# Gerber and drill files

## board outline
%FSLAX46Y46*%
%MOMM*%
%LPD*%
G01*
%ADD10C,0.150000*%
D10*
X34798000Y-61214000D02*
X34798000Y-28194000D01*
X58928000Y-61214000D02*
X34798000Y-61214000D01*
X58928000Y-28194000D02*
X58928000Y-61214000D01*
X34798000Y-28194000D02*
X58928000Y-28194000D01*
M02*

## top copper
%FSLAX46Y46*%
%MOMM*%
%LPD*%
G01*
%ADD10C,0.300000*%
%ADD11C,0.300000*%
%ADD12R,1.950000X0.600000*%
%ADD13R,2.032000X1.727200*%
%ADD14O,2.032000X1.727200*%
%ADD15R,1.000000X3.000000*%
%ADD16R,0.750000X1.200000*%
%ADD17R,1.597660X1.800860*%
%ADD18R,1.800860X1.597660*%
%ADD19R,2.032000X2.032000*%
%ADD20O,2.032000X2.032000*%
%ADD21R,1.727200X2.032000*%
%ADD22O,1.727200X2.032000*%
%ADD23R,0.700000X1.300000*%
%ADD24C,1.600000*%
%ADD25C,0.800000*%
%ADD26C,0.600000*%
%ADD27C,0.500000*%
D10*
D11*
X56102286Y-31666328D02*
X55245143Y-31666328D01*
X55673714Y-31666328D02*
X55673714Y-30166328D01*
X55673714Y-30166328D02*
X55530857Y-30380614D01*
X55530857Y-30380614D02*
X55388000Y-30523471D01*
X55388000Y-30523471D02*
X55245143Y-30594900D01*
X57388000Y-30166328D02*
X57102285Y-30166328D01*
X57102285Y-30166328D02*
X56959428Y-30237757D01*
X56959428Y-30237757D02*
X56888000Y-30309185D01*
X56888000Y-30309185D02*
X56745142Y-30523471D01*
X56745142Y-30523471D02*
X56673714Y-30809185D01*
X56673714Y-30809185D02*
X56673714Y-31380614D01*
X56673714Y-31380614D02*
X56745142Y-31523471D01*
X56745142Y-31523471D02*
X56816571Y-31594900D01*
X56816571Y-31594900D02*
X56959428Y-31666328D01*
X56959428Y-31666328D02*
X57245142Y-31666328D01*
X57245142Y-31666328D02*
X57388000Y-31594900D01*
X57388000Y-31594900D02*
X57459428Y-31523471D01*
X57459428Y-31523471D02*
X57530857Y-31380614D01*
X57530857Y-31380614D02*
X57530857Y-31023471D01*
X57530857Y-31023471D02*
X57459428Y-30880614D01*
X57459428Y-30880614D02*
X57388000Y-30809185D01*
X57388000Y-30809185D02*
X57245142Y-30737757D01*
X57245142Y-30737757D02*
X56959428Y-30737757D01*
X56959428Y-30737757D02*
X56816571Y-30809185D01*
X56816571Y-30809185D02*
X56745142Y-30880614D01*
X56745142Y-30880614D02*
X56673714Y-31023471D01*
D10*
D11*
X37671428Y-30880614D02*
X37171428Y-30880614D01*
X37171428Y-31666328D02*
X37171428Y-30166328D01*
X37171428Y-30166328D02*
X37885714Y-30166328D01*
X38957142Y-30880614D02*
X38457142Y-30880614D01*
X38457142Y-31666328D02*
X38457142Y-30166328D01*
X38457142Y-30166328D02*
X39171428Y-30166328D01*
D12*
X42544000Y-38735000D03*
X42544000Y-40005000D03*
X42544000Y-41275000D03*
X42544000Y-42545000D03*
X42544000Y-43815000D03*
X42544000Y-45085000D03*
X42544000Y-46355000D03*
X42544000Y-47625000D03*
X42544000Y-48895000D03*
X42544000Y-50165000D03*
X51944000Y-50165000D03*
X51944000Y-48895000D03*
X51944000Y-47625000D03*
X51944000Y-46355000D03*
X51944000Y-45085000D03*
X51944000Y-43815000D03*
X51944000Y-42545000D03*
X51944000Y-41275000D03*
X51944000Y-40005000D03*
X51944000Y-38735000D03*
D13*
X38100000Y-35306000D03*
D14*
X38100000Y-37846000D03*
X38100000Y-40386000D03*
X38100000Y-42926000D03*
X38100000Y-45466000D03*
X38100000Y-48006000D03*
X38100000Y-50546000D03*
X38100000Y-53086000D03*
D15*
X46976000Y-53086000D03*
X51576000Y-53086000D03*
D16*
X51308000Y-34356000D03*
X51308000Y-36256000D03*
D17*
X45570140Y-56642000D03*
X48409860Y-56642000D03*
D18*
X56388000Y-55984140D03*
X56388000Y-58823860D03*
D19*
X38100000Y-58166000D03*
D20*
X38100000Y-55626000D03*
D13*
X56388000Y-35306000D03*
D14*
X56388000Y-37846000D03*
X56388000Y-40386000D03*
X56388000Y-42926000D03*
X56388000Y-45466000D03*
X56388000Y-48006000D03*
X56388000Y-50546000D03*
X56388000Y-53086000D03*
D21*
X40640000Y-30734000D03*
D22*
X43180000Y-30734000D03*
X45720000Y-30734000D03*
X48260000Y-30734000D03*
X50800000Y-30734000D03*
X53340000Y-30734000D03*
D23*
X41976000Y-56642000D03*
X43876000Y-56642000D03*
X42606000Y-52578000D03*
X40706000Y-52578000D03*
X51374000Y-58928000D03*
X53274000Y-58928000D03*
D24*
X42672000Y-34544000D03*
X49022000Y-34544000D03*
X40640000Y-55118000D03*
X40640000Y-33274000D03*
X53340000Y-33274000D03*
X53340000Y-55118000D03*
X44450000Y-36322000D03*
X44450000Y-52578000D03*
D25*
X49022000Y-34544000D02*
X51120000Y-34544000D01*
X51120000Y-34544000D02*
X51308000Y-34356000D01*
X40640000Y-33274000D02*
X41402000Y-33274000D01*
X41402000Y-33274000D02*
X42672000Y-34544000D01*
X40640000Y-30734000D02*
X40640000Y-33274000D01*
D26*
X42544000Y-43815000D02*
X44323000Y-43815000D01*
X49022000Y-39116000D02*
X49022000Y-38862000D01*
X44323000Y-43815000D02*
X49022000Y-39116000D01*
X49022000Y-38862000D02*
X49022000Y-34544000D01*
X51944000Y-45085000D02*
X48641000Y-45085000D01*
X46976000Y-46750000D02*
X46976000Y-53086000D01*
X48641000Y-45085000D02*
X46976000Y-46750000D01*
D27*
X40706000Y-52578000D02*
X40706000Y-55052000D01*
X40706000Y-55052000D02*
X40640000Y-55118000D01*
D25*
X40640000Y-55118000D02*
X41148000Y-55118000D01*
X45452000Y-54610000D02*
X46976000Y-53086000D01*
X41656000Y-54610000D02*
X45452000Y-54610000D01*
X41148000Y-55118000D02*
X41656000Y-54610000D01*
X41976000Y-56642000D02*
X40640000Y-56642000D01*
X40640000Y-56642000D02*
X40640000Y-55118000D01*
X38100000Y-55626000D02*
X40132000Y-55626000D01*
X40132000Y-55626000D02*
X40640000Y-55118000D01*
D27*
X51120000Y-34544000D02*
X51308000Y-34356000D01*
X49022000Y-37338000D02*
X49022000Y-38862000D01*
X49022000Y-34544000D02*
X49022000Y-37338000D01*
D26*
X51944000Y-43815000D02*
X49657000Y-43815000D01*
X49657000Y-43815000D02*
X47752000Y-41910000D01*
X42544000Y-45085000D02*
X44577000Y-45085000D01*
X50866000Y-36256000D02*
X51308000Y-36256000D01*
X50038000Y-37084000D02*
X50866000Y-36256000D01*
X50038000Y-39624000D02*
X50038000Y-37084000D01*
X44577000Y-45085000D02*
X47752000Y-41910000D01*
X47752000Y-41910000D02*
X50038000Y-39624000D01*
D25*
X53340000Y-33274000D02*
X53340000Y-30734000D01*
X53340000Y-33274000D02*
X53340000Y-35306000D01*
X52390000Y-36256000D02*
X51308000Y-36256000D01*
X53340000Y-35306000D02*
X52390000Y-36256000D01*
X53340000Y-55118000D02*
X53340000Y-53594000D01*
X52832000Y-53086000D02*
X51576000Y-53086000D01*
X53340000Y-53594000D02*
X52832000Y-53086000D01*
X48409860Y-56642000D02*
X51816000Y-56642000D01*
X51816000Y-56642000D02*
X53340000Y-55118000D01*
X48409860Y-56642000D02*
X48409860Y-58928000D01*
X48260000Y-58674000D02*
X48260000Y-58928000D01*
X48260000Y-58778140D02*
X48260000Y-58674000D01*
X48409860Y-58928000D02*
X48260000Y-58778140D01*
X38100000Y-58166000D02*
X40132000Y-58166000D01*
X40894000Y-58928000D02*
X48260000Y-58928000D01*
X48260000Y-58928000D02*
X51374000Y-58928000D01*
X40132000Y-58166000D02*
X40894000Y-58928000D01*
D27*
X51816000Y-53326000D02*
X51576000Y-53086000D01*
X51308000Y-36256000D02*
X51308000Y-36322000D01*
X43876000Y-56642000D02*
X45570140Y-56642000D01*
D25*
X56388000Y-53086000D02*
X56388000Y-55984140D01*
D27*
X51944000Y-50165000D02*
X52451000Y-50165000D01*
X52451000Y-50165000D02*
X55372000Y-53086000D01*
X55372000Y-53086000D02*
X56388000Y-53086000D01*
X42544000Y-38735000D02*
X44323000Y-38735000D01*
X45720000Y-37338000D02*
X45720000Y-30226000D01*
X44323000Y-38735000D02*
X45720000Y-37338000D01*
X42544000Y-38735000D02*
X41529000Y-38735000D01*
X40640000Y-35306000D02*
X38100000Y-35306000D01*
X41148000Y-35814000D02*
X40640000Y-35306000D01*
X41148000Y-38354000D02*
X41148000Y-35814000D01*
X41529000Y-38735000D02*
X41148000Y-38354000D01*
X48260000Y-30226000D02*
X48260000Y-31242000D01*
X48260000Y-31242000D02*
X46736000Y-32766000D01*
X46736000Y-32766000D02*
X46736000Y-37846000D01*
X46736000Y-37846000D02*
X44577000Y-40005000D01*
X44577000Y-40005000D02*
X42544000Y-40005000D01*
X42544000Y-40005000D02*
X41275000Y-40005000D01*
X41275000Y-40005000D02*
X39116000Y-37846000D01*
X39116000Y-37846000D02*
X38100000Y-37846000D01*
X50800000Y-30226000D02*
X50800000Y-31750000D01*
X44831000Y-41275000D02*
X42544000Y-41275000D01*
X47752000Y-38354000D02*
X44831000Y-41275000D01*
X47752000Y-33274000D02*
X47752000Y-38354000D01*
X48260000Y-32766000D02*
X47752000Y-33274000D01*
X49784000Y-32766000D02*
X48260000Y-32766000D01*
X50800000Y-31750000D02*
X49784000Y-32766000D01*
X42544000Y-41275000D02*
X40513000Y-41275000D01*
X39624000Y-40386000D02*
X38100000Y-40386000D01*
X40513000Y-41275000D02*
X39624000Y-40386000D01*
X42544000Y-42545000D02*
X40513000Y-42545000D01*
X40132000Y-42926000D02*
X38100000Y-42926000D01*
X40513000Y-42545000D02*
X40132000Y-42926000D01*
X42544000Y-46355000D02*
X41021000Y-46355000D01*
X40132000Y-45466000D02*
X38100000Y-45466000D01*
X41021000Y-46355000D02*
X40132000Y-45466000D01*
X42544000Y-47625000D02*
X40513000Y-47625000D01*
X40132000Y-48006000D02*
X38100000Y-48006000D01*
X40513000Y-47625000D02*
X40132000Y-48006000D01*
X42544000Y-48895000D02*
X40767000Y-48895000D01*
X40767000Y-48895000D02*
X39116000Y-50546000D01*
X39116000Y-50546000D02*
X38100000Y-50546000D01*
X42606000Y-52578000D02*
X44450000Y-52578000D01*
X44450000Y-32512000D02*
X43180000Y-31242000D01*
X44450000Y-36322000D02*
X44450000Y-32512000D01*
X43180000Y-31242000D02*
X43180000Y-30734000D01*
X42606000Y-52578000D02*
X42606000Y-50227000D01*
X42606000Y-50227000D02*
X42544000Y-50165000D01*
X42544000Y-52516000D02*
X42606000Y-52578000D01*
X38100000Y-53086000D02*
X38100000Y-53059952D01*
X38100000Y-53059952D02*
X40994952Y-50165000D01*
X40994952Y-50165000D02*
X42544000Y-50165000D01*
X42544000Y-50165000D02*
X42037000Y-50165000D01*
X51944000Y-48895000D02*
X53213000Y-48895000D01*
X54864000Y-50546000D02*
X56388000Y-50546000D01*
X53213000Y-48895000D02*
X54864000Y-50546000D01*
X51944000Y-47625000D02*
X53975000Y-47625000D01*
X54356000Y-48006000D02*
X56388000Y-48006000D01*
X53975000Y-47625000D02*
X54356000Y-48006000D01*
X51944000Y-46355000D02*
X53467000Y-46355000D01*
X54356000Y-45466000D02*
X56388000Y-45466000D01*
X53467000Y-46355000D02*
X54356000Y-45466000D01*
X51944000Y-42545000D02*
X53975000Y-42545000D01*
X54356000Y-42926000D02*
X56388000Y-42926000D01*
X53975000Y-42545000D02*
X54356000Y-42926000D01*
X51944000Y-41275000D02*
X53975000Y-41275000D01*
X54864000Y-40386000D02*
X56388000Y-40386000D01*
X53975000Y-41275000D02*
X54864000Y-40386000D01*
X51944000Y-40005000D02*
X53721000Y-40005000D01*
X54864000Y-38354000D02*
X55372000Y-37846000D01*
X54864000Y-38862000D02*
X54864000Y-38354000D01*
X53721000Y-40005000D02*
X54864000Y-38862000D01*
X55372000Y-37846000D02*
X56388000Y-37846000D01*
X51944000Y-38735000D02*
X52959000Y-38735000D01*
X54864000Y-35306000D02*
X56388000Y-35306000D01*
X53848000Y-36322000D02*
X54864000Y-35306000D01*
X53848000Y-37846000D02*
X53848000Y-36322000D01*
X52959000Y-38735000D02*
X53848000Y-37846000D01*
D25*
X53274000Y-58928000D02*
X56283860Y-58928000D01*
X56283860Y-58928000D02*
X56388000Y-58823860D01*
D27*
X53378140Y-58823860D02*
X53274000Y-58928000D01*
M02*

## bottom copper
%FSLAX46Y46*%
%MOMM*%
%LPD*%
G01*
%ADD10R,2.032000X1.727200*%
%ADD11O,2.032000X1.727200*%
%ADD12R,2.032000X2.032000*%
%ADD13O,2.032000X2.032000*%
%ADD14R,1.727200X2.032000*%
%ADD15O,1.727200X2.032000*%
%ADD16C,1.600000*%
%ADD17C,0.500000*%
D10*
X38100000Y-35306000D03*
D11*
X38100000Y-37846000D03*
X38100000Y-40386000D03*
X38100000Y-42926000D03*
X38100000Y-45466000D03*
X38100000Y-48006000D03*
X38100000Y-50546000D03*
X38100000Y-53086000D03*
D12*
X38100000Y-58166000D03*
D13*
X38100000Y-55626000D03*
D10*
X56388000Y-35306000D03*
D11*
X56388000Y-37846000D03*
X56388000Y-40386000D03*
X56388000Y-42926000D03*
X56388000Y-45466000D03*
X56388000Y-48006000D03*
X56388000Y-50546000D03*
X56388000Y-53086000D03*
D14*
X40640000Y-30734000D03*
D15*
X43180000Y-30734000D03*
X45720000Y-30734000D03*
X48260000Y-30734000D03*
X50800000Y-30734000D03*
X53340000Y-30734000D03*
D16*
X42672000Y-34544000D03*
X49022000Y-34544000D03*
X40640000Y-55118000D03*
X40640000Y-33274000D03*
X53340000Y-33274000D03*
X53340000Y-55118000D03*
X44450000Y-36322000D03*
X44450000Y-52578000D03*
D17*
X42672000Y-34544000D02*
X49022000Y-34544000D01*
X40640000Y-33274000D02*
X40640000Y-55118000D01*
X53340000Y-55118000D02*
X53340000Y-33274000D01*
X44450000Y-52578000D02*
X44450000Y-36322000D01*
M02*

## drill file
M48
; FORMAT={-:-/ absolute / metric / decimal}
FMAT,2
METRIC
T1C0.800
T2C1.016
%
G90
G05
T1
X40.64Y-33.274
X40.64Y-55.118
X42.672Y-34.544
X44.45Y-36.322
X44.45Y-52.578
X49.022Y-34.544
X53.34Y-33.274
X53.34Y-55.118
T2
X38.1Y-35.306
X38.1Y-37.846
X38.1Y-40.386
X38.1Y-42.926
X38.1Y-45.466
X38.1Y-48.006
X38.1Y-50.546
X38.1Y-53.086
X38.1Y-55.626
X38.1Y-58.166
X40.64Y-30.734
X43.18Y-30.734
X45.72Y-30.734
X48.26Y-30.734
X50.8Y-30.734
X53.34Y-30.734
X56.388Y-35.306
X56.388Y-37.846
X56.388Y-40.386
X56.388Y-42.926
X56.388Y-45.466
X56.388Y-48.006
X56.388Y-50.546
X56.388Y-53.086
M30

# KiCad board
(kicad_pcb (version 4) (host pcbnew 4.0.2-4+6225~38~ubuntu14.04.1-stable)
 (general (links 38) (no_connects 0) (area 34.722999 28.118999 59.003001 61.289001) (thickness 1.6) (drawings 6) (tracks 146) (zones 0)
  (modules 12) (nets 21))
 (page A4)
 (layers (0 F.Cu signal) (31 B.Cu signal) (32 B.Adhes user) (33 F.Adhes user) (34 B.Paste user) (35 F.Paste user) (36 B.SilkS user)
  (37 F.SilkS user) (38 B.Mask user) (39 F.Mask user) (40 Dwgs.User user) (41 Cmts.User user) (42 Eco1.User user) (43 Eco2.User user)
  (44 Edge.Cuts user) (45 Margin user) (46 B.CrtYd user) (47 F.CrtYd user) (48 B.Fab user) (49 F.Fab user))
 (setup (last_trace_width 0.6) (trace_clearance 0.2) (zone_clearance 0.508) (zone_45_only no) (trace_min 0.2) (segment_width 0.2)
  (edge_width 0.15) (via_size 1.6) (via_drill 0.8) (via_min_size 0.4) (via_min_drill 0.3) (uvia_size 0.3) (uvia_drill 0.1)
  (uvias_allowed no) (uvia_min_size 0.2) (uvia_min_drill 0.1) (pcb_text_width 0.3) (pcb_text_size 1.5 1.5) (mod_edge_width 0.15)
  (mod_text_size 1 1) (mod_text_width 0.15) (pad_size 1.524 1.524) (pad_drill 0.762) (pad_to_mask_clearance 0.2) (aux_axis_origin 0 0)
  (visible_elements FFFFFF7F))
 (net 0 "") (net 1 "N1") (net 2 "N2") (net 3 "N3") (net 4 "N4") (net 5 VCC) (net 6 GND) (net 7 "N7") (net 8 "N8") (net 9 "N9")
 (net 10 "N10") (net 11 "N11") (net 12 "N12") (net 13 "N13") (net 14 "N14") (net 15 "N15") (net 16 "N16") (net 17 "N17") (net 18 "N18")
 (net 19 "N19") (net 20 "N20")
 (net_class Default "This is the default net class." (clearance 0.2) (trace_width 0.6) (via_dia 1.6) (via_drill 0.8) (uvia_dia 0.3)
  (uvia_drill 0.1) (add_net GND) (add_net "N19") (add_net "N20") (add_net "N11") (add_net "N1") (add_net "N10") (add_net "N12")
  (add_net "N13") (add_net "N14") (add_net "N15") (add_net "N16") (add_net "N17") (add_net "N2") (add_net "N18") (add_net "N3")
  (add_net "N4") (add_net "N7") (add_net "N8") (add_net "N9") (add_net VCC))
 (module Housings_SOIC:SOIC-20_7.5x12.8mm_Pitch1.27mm (layer F.Cu) (at 47.244 44.45)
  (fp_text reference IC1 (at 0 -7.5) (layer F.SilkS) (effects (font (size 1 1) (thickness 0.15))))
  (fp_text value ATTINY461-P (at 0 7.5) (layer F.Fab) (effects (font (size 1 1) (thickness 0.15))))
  (pad 1 smd rect (at -4.7 -5.715) (size 1.95 0.6) (layers F.Cu F.Paste F.Mask) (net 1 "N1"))
  (pad 2 smd rect (at -4.7 -4.445) (size 1.95 0.6) (layers F.Cu F.Paste F.Mask) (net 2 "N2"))
  (pad 3 smd rect (at -4.7 -3.175) (size 1.95 0.6) (layers F.Cu F.Paste F.Mask) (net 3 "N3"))
  (pad 4 smd rect (at -4.7 -1.905) (size 1.95 0.6) (layers F.Cu F.Paste F.Mask) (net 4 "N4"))
  (pad 5 smd rect (at -4.7 -0.635) (size 1.95 0.6) (layers F.Cu F.Paste F.Mask) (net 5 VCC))
  (pad 6 smd rect (at -4.7 0.635) (size 1.95 0.6) (layers F.Cu F.Paste F.Mask) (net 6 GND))
  (pad 7 smd rect (at -4.7 1.905) (size 1.95 0.6) (layers F.Cu F.Paste F.Mask) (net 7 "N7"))
  (pad 8 smd rect (at -4.7 3.175) (size 1.95 0.6) (layers F.Cu F.Paste F.Mask) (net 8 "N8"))
  (pad 9 smd rect (at -4.7 4.445) (size 1.95 0.6) (layers F.Cu F.Paste F.Mask) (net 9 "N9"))
  (pad 10 smd rect (at -4.7 5.715) (size 1.95 0.6) (layers F.Cu F.Paste F.Mask) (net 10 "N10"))
  (pad 11 smd rect (at 4.7 5.715) (size 1.95 0.6) (layers F.Cu F.Paste F.Mask) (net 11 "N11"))
  (pad 12 smd rect (at 4.7 4.445) (size 1.95 0.6) (layers F.Cu F.Paste F.Mask) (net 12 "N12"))
  (pad 13 smd rect (at 4.7 3.175) (size 1.95 0.6) (layers F.Cu F.Paste F.Mask) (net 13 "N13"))
  (pad 14 smd rect (at 4.7 1.905) (size 1.95 0.6) (layers F.Cu F.Paste F.Mask) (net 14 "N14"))
  (pad 15 smd rect (at 4.7 0.635) (size 1.95 0.6) (layers F.Cu F.Paste F.Mask) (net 5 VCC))
  (pad 16 smd rect (at 4.7 -0.635) (size 1.95 0.6) (layers F.Cu F.Paste F.Mask) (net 6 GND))
  (pad 17 smd rect (at 4.7 -1.905) (size 1.95 0.6) (layers F.Cu F.Paste F.Mask) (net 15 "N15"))
  (pad 18 smd rect (at 4.7 -3.175) (size 1.95 0.6) (layers F.Cu F.Paste F.Mask) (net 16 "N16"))
  (pad 19 smd rect (at 4.7 -4.445) (size 1.95 0.6) (layers F.Cu F.Paste F.Mask) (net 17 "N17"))
  (pad 20 smd rect (at 4.7 -5.715) (size 1.95 0.6) (layers F.Cu F.Paste F.Mask) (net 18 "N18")))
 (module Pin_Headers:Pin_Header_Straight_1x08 (layer F.Cu) (at 38.1 35.306)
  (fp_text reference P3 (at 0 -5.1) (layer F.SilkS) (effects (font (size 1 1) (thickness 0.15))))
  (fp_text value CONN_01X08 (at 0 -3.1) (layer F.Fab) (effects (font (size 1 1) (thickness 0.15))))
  (pad 1 thru_hole rect (at 0 0) (size 2.032 1.7272) (drill 1.016) (layers *.Cu *.Mask F.SilkS) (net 1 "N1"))
  (pad 2 thru_hole oval (at 0 2.54) (size 2.032 1.7272) (drill 1.016) (layers *.Cu *.Mask F.SilkS) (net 2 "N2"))
  (pad 3 thru_hole oval (at 0 5.08) (size 2.032 1.7272) (drill 1.016) (layers *.Cu *.Mask F.SilkS) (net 3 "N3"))
  (pad 4 thru_hole oval (at 0 7.62) (size 2.032 1.7272) (drill 1.016) (layers *.Cu *.Mask F.SilkS) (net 4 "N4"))
  (pad 5 thru_hole oval (at 0 10.16) (size 2.032 1.7272) (drill 1.016) (layers *.Cu *.Mask F.SilkS) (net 7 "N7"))
  (pad 6 thru_hole oval (at 0 12.7) (size 2.032 1.7272) (drill 1.016) (layers *.Cu *.Mask F.SilkS) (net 8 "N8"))
  (pad 7 thru_hole oval (at 0 15.24) (size 2.032 1.7272) (drill 1.016) (layers *.Cu *.Mask F.SilkS) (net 9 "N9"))
  (pad 8 thru_hole oval (at 0 17.78) (size 2.032 1.7272) (drill 1.016) (layers *.Cu *.Mask F.SilkS) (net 10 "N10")))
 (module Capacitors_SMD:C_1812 (layer F.Cu) (at 49.276 53.086)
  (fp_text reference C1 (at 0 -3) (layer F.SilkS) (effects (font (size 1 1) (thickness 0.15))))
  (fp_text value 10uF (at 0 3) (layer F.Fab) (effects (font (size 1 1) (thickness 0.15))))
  (pad 1 smd rect (at -2.3 0) (size 1 3) (layers F.Cu F.Paste F.Mask) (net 5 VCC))
  (pad 2 smd rect (at 2.3 0) (size 1 3) (layers F.Cu F.Paste F.Mask) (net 6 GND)))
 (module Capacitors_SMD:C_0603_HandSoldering (layer F.Cu) (at 51.308 35.306 270)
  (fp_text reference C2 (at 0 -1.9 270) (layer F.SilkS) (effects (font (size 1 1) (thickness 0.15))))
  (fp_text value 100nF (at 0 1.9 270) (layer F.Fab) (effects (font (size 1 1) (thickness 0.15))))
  (pad 1 smd rect (at -0.95 0 270) (size 1.2 0.75) (layers F.Cu F.Paste F.Mask) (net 5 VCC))
  (pad 2 smd rect (at 0.95 0 270) (size 1.2 0.75) (layers F.Cu F.Paste F.Mask) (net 6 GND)))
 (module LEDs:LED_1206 (layer F.Cu) (at 46.99 56.642 180)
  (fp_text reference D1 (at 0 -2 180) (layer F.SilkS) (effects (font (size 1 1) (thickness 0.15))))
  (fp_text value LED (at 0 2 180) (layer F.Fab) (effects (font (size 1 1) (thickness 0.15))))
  (pad 2 smd rect (at 1.41986 0) (size 1.59766 1.80086) (layers F.Cu F.Paste F.Mask) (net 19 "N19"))
  (pad 1 smd rect (at -1.41986 0) (size 1.59766 1.80086) (layers F.Cu F.Paste F.Mask) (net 6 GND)))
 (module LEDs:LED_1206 (layer F.Cu) (at 56.388 57.404 90)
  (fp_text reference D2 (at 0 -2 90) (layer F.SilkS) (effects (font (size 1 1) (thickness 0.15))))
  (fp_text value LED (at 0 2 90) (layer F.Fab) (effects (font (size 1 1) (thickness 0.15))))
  (pad 2 smd rect (at 1.41986 0 270) (size 1.59766 1.80086) (layers F.Cu F.Paste F.Mask) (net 11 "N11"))
  (pad 1 smd rect (at -1.41986 0 270) (size 1.59766 1.80086) (layers F.Cu F.Paste F.Mask) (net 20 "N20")))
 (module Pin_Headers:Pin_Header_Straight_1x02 (layer F.Cu) (at 38.1 58.166 180)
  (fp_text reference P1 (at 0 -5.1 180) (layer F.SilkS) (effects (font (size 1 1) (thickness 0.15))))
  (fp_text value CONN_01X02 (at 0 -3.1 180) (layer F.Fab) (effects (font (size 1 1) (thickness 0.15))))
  (pad 1 thru_hole rect (at 0 0 180) (size 2.032 2.032) (drill 1.016) (layers *.Cu *.Mask F.SilkS) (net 6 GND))
  (pad 2 thru_hole oval (at 0 2.54 180) (size 2.032 2.032) (drill 1.016) (layers *.Cu *.Mask F.SilkS) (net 5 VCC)))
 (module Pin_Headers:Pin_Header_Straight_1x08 (layer F.Cu) (at 56.388 35.306)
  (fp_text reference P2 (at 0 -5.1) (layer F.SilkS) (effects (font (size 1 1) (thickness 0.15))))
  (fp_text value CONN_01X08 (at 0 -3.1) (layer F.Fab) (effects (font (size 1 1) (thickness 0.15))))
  (pad 1 thru_hole rect (at 0 0) (size 2.032 1.7272) (drill 1.016) (layers *.Cu *.Mask F.SilkS) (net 18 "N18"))
  (pad 2 thru_hole oval (at 0 2.54) (size 2.032 1.7272) (drill 1.016) (layers *.Cu *.Mask F.SilkS) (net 17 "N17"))
  (pad 3 thru_hole oval (at 0 5.08) (size 2.032 1.7272) (drill 1.016) (layers *.Cu *.Mask F.SilkS) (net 16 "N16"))
  (pad 4 thru_hole oval (at 0 7.62) (size 2.032 1.7272) (drill 1.016) (layers *.Cu *.Mask F.SilkS) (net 15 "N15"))
  (pad 5 thru_hole oval (at 0 10.16) (size 2.032 1.7272) (drill 1.016) (layers *.Cu *.Mask F.SilkS) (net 14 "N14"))
  (pad 6 thru_hole oval (at 0 12.7) (size 2.032 1.7272) (drill 1.016) (layers *.Cu *.Mask F.SilkS) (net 13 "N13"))
  (pad 7 thru_hole oval (at 0 15.24) (size 2.032 1.7272) (drill 1.016) (layers *.Cu *.Mask F.SilkS) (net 12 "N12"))
  (pad 8 thru_hole oval (at 0 17.78) (size 2.032 1.7272) (drill 1.016) (layers *.Cu *.Mask F.SilkS) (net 11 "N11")))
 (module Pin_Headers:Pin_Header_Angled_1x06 (layer F.Cu) (at 40.64 30.734 90)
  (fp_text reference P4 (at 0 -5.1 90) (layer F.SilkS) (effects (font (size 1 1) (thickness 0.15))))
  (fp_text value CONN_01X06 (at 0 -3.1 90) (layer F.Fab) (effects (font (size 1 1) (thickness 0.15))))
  (pad 1 thru_hole rect (at 0 0 90) (size 2.032 1.7272) (drill 1.016) (layers *.Cu *.Mask F.SilkS) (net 5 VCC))
  (pad 2 thru_hole oval (at 0 2.54 90) (size 2.032 1.7272) (drill 1.016) (layers *.Cu *.Mask F.SilkS) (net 10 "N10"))
  (pad 3 thru_hole oval (at 0 5.08 90) (size 2.032 1.7272) (drill 1.016) (layers *.Cu *.Mask F.SilkS) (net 1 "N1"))
  (pad 4 thru_hole oval (at 0 7.62 90) (size 2.032 1.7272) (drill 1.016) (layers *.Cu *.Mask F.SilkS) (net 2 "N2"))
  (pad 5 thru_hole oval (at 0 10.16 90) (size 2.032 1.7272) (drill 1.016) (layers *.Cu *.Mask F.SilkS) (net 3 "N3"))
  (pad 6 thru_hole oval (at 0 12.7 90) (size 2.032 1.7272) (drill 1.016) (layers *.Cu *.Mask F.SilkS) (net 6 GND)))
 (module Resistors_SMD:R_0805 (layer F.Cu) (at 42.926 56.642)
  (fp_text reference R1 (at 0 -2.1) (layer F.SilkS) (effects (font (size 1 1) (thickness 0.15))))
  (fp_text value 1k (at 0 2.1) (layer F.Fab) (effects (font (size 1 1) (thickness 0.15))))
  (pad 1 smd rect (at -0.95 0) (size 0.7 1.3) (layers F.Cu F.Paste F.Mask) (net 5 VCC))
  (pad 2 smd rect (at 0.95 0) (size 0.7 1.3) (layers F.Cu F.Paste F.Mask) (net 19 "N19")))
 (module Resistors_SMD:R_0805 (layer F.Cu) (at 41.656 52.578 180)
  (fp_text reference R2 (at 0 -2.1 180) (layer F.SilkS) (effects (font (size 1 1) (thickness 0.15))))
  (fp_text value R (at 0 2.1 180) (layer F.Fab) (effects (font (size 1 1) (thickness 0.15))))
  (pad 1 smd rect (at -0.95 0 180) (size 0.7 1.3) (layers F.Cu F.Paste F.Mask) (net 10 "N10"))
  (pad 2 smd rect (at 0.95 0 180) (size 0.7 1.3) (layers F.Cu F.Paste F.Mask) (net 5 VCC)))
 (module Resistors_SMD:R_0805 (layer F.Cu) (at 52.324 58.928)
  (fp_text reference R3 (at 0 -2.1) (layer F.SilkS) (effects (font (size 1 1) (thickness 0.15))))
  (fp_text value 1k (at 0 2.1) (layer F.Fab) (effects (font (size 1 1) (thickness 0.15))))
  (pad 1 smd rect (at -0.95 0) (size 0.7 1.3) (layers F.Cu F.Paste F.Mask) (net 6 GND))
  (pad 2 smd rect (at 0.95 0) (size 0.7 1.3) (layers F.Cu F.Paste F.Mask) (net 20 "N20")))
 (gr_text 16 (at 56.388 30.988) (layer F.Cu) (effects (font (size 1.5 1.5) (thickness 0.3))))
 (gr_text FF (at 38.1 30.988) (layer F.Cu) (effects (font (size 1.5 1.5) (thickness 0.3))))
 (gr_line (start 34.798 61.214) (end 34.798 28.194) (angle 90) (layer Edge.Cuts) (width 0.15))
 (gr_line (start 58.928 61.214) (end 34.798 61.214) (angle 90) (layer Edge.Cuts) (width 0.15))
 (gr_line (start 58.928 28.194) (end 58.928 61.214) (angle 90) (layer Edge.Cuts) (width 0.15))
 (gr_line (start 34.798 28.194) (end 58.928 28.194) (angle 90) (layer Edge.Cuts) (width 0.15))
 (segment (start 49.022 34.544) (end 51.12 34.544) (width 0.8) (layer F.Cu) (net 5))
 (segment (start 51.12 34.544) (end 51.308 34.356) (width 0.8) (layer F.Cu) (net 5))
 (segment (start 40.64 33.274) (end 41.402 33.274) (width 0.8) (layer F.Cu) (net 5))
 (segment (start 42.672 34.544) (end 49.022 34.544) (width 0.5) (layer B.Cu) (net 5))
 (segment (start 41.402 33.274) (end 42.672 34.544) (width 0.8) (layer F.Cu) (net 5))
 (segment (start 40.64 30.734) (end 40.64 33.274) (width 0.8) (layer F.Cu) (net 5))
 (segment (start 40.64 33.274) (end 40.64 55.118) (width 0.5) (layer B.Cu) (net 5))
 (segment (start 42.544 43.815) (end 44.323 43.815) (width 0.6) (layer F.Cu) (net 5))
 (segment (start 49.022 39.116) (end 49.022 38.862) (width 0.6) (layer F.Cu) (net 5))
 (segment (start 44.323 43.815) (end 49.022 39.116) (width 0.6) (layer F.Cu) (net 5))
 (segment (start 49.022 38.862) (end 49.022 34.544) (width 0.6) (layer F.Cu) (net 5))
 (segment (start 51.944 45.085) (end 48.641 45.085) (width 0.6) (layer F.Cu) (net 5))
 (segment (start 46.976 46.75) (end 46.976 53.086) (width 0.6) (layer F.Cu) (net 5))
 (segment (start 48.641 45.085) (end 46.976 46.75) (width 0.6) (layer F.Cu) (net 5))
 (segment (start 40.706 52.578) (end 40.706 55.052) (width 0.5) (layer F.Cu) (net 5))
 (segment (start 40.706 55.052) (end 40.64 55.118) (width 0.5) (layer F.Cu) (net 5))
 (segment (start 40.64 55.118) (end 41.148 55.118) (width 0.8) (layer F.Cu) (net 5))
 (segment (start 45.452 54.61) (end 46.976 53.086) (width 0.8) (layer F.Cu) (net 5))
 (segment (start 41.656 54.61) (end 45.452 54.61) (width 0.8) (layer F.Cu) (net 5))
 (segment (start 41.148 55.118) (end 41.656 54.61) (width 0.8) (layer F.Cu) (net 5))
 (segment (start 41.976 56.642) (end 40.64 56.642) (width 0.8) (layer F.Cu) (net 5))
 (segment (start 40.64 56.642) (end 40.64 55.118) (width 0.8) (layer F.Cu) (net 5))
 (segment (start 38.1 55.626) (end 40.132 55.626) (width 0.8) (layer F.Cu) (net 5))
 (segment (start 40.132 55.626) (end 40.64 55.118) (width 0.8) (layer F.Cu) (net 5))
 (segment (start 51.12 34.544) (end 51.308 34.356) (width 0.5) (layer F.Cu) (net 5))
 (segment (start 49.022 37.338) (end 49.022 38.862) (width 0.5) (layer F.Cu) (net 5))
 (segment (start 49.022 34.544) (end 49.022 37.338) (width 0.5) (layer F.Cu) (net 5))
 (segment (start 51.944 43.815) (end 49.657 43.815) (width 0.6) (layer F.Cu) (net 6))
 (segment (start 49.657 43.815) (end 47.752 41.91) (width 0.6) (layer F.Cu) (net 6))
 (segment (start 42.544 45.085) (end 44.577 45.085) (width 0.6) (layer F.Cu) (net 6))
 (segment (start 50.866 36.256) (end 51.308 36.256) (width 0.6) (layer F.Cu) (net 6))
 (segment (start 50.038 37.084) (end 50.866 36.256) (width 0.6) (layer F.Cu) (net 6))
 (segment (start 50.038 39.624) (end 50.038 37.084) (width 0.6) (layer F.Cu) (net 6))
 (segment (start 44.577 45.085) (end 47.752 41.91) (width 0.6) (layer F.Cu) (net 6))
 (segment (start 47.752 41.91) (end 50.038 39.624) (width 0.6) (layer F.Cu) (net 6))
 (segment (start 53.34 33.274) (end 53.34 30.734) (width 0.8) (layer F.Cu) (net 6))
 (segment (start 53.34 33.274) (end 53.34 35.306) (width 0.8) (layer F.Cu) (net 6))
 (segment (start 53.34 55.118) (end 53.34 33.274) (width 0.5) (layer B.Cu) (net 6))
 (segment (start 52.39 36.256) (end 51.308 36.256) (width 0.8) (layer F.Cu) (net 6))
 (segment (start 53.34 35.306) (end 52.39 36.256) (width 0.8) (layer F.Cu) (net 6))
 (segment (start 53.34 55.118) (end 53.34 53.594) (width 0.8) (layer F.Cu) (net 6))
 (segment (start 52.832 53.086) (end 51.576 53.086) (width 0.8) (layer F.Cu) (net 6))
 (segment (start 53.34 53.594) (end 52.832 53.086) (width 0.8) (layer F.Cu) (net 6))
 (segment (start 48.40986 56.642) (end 51.816 56.642) (width 0.8) (layer F.Cu) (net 6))
 (segment (start 51.816 56.642) (end 53.34 55.118) (width 0.8) (layer F.Cu) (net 6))
 (segment (start 48.40986 56.642) (end 48.40986 58.928) (width 0.8) (layer F.Cu) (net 6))
 (segment (start 48.26 58.674) (end 48.26 58.928) (width 0.8) (layer F.Cu) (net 6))
 (segment (start 48.26 58.77814) (end 48.26 58.674) (width 0.8) (layer F.Cu) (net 6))
 (segment (start 48.40986 58.928) (end 48.26 58.77814) (width 0.8) (layer F.Cu) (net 6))
 (segment (start 38.1 58.166) (end 40.132 58.166) (width 0.8) (layer F.Cu) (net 6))
 (segment (start 40.894 58.928) (end 48.26 58.928) (width 0.8) (layer F.Cu) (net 6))
 (segment (start 48.26 58.928) (end 51.374 58.928) (width 0.8) (layer F.Cu) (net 6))
 (segment (start 40.132 58.166) (end 40.894 58.928) (width 0.8) (layer F.Cu) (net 6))
 (segment (start 51.816 53.326) (end 51.576 53.086) (width 0.5) (layer F.Cu) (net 6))
 (segment (start 51.308 36.256) (end 51.308 36.322) (width 0.5) (layer F.Cu) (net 6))
 (segment (start 43.876 56.642) (end 45.57014 56.642) (width 0.5) (layer F.Cu) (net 19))
 (segment (start 56.388 53.086) (end 56.388 55.98414) (width 0.8) (layer F.Cu) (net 11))
 (segment (start 51.944 50.165) (end 52.451 50.165) (width 0.5) (layer F.Cu) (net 11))
 (segment (start 52.451 50.165) (end 55.372 53.086) (width 0.5) (layer F.Cu) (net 11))
 (segment (start 55.372 53.086) (end 56.388 53.086) (width 0.5) (layer F.Cu) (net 11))
 (segment (start 42.544 38.735) (end 44.323 38.735) (width 0.5) (layer F.Cu) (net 1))
 (segment (start 45.72 37.338) (end 45.72 30.226) (width 0.5) (layer F.Cu) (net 1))
 (segment (start 44.323 38.735) (end 45.72 37.338) (width 0.5) (layer F.Cu) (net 1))
 (segment (start 42.544 38.735) (end 41.529 38.735) (width 0.5) (layer F.Cu) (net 1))
 (segment (start 40.64 35.306) (end 38.1 35.306) (width 0.5) (layer F.Cu) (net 1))
 (segment (start 41.148 35.814) (end 40.64 35.306) (width 0.5) (layer F.Cu) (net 1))
 (segment (start 41.148 38.354) (end 41.148 35.814) (width 0.5) (layer F.Cu) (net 1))
 (segment (start 41.529 38.735) (end 41.148 38.354) (width 0.5) (layer F.Cu) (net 1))
 (segment (start 48.26 30.226) (end 48.26 31.242) (width 0.5) (layer F.Cu) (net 2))
 (segment (start 48.26 31.242) (end 46.736 32.766) (width 0.5) (layer F.Cu) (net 2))
 (segment (start 46.736 32.766) (end 46.736 37.846) (width 0.5) (layer F.Cu) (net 2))
 (segment (start 46.736 37.846) (end 44.577 40.005) (width 0.5) (layer F.Cu) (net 2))
 (segment (start 44.577 40.005) (end 42.544 40.005) (width 0.5) (layer F.Cu) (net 2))
 (segment (start 42.544 40.005) (end 41.275 40.005) (width 0.5) (layer F.Cu) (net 2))
 (segment (start 41.275 40.005) (end 39.116 37.846) (width 0.5) (layer F.Cu) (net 2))
 (segment (start 39.116 37.846) (end 38.1 37.846) (width 0.5) (layer F.Cu) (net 2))
 (segment (start 50.8 30.226) (end 50.8 31.75) (width 0.5) (layer F.Cu) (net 3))
 (segment (start 44.831 41.275) (end 42.544 41.275) (width 0.5) (layer F.Cu) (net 3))
 (segment (start 47.752 38.354) (end 44.831 41.275) (width 0.5) (layer F.Cu) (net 3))
 (segment (start 47.752 33.274) (end 47.752 38.354) (width 0.5) (layer F.Cu) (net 3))
 (segment (start 48.26 32.766) (end 47.752 33.274) (width 0.5) (layer F.Cu) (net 3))
 (segment (start 49.784 32.766) (end 48.26 32.766) (width 0.5) (layer F.Cu) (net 3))
 (segment (start 50.8 31.75) (end 49.784 32.766) (width 0.5) (layer F.Cu) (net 3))
 (segment (start 42.544 41.275) (end 40.513 41.275) (width 0.5) (layer F.Cu) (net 3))
 (segment (start 39.624 40.386) (end 38.1 40.386) (width 0.5) (layer F.Cu) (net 3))
 (segment (start 40.513 41.275) (end 39.624 40.386) (width 0.5) (layer F.Cu) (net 3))
 (segment (start 42.544 42.545) (end 40.513 42.545) (width 0.5) (layer F.Cu) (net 4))
 (segment (start 40.132 42.926) (end 38.1 42.926) (width 0.5) (layer F.Cu) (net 4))
 (segment (start 40.513 42.545) (end 40.132 42.926) (width 0.5) (layer F.Cu) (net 4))
 (segment (start 42.544 46.355) (end 41.021 46.355) (width 0.5) (layer F.Cu) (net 7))
 (segment (start 40.132 45.466) (end 38.1 45.466) (width 0.5) (layer F.Cu) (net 7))
 (segment (start 41.021 46.355) (end 40.132 45.466) (width 0.5) (layer F.Cu) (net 7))
 (segment (start 42.544 47.625) (end 40.513 47.625) (width 0.5) (layer F.Cu) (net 8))
 (segment (start 40.132 48.006) (end 38.1 48.006) (width 0.5) (layer F.Cu) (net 8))
 (segment (start 40.513 47.625) (end 40.132 48.006) (width 0.5) (layer F.Cu) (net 8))
 (segment (start 42.544 48.895) (end 40.767 48.895) (width 0.5) (layer F.Cu) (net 9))
 (segment (start 40.767 48.895) (end 39.116 50.546) (width 0.5) (layer F.Cu) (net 9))
 (segment (start 39.116 50.546) (end 38.1 50.546) (width 0.5) (layer F.Cu) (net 9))
 (segment (start 42.606 52.578) (end 44.45 52.578) (width 0.5) (layer F.Cu) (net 10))
 (segment (start 44.45 32.512) (end 43.18 31.242) (width 0.5) (layer F.Cu) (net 10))
 (segment (start 44.45 36.322) (end 44.45 32.512) (width 0.5) (layer F.Cu) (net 10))
 (segment (start 44.45 52.578) (end 44.45 36.322) (width 0.5) (layer B.Cu) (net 10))
 (segment (start 43.18 31.242) (end 43.18 30.734) (width 0.5) (layer F.Cu) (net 10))
 (segment (start 42.606 52.578) (end 42.606 50.227) (width 0.5) (layer F.Cu) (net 10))
 (segment (start 42.606 50.227) (end 42.544 50.165) (width 0.5) (layer F.Cu) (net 10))
 (segment (start 42.544 52.516) (end 42.606 52.578) (width 0.5) (layer F.Cu) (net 10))
 (segment (start 38.1 53.086) (end 38.1 53.059952) (width 0.5) (layer F.Cu) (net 10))
 (segment (start 38.1 53.059952) (end 40.994952 50.165) (width 0.5) (layer F.Cu) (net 10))
 (segment (start 40.994952 50.165) (end 42.544 50.165) (width 0.5) (layer F.Cu) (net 10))
 (segment (start 42.544 50.165) (end 42.037 50.165) (width 0.5) (layer F.Cu) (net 10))
 (segment (start 51.944 48.895) (end 53.213 48.895) (width 0.5) (layer F.Cu) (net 12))
 (segment (start 54.864 50.546) (end 56.388 50.546) (width 0.5) (layer F.Cu) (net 12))
 (segment (start 53.213 48.895) (end 54.864 50.546) (width 0.5) (layer F.Cu) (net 12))
 (segment (start 51.944 47.625) (end 53.975 47.625) (width 0.5) (layer F.Cu) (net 13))
 (segment (start 54.356 48.006) (end 56.388 48.006) (width 0.5) (layer F.Cu) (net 13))
 (segment (start 53.975 47.625) (end 54.356 48.006) (width 0.5) (layer F.Cu) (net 13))
 (segment (start 51.944 46.355) (end 53.467 46.355) (width 0.5) (layer F.Cu) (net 14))
 (segment (start 54.356 45.466) (end 56.388 45.466) (width 0.5) (layer F.Cu) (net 14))
 (segment (start 53.467 46.355) (end 54.356 45.466) (width 0.5) (layer F.Cu) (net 14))
 (segment (start 51.944 42.545) (end 53.975 42.545) (width 0.5) (layer F.Cu) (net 15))
 (segment (start 54.356 42.926) (end 56.388 42.926) (width 0.5) (layer F.Cu) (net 15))
 (segment (start 53.975 42.545) (end 54.356 42.926) (width 0.5) (layer F.Cu) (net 15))
 (segment (start 51.944 41.275) (end 53.975 41.275) (width 0.5) (layer F.Cu) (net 16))
 (segment (start 54.864 40.386) (end 56.388 40.386) (width 0.5) (layer F.Cu) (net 16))
 (segment (start 53.975 41.275) (end 54.864 40.386) (width 0.5) (layer F.Cu) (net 16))
 (segment (start 51.944 40.005) (end 53.721 40.005) (width 0.5) (layer F.Cu) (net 17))
 (segment (start 54.864 38.354) (end 55.372 37.846) (width 0.5) (layer F.Cu) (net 17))
 (segment (start 54.864 38.862) (end 54.864 38.354) (width 0.5) (layer F.Cu) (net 17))
 (segment (start 53.721 40.005) (end 54.864 38.862) (width 0.5) (layer F.Cu) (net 17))
 (segment (start 55.372 37.846) (end 56.388 37.846) (width 0.5) (layer F.Cu) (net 17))
 (segment (start 51.944 38.735) (end 52.959 38.735) (width 0.5) (layer F.Cu) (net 18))
 (segment (start 54.864 35.306) (end 56.388 35.306) (width 0.5) (layer F.Cu) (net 18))
 (segment (start 53.848 36.322) (end 54.864 35.306) (width 0.5) (layer F.Cu) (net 18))
 (segment (start 53.848 37.846) (end 53.848 36.322) (width 0.5) (layer F.Cu) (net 18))
 (segment (start 52.959 38.735) (end 53.848 37.846) (width 0.5) (layer F.Cu) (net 18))
 (segment (start 53.274 58.928) (end 56.28386 58.928) (width 0.8) (layer F.Cu) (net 20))
 (segment (start 56.28386 58.928) (end 56.388 58.82386) (width 0.8) (layer F.Cu) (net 20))
 (segment (start 53.37814 58.82386) (end 53.274 58.928) (width 0.5) (layer F.Cu) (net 20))
 (via (at 42.672 34.544) (size 1.6) (drill 0.8) (layers F.Cu B.Cu) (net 5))
 (via (at 49.022 34.544) (size 1.6) (drill 0.8) (layers F.Cu B.Cu) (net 5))
 (via (at 40.64 55.118) (size 1.6) (drill 0.8) (layers F.Cu B.Cu) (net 5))
 (via (at 40.64 33.274) (size 1.6) (drill 0.8) (layers F.Cu B.Cu) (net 5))
 (via (at 53.34 33.274) (size 1.6) (drill 0.8) (layers F.Cu B.Cu) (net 6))
 (via (at 53.34 55.118) (size 1.6) (drill 0.8) (layers F.Cu B.Cu) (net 6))
 (via (at 44.45 36.322) (size 1.6) (drill 0.8) (layers F.Cu B.Cu) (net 10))
 (via (at 44.45 52.578) (size 1.6) (drill 0.8) (layers F.Cu B.Cu) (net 10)))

